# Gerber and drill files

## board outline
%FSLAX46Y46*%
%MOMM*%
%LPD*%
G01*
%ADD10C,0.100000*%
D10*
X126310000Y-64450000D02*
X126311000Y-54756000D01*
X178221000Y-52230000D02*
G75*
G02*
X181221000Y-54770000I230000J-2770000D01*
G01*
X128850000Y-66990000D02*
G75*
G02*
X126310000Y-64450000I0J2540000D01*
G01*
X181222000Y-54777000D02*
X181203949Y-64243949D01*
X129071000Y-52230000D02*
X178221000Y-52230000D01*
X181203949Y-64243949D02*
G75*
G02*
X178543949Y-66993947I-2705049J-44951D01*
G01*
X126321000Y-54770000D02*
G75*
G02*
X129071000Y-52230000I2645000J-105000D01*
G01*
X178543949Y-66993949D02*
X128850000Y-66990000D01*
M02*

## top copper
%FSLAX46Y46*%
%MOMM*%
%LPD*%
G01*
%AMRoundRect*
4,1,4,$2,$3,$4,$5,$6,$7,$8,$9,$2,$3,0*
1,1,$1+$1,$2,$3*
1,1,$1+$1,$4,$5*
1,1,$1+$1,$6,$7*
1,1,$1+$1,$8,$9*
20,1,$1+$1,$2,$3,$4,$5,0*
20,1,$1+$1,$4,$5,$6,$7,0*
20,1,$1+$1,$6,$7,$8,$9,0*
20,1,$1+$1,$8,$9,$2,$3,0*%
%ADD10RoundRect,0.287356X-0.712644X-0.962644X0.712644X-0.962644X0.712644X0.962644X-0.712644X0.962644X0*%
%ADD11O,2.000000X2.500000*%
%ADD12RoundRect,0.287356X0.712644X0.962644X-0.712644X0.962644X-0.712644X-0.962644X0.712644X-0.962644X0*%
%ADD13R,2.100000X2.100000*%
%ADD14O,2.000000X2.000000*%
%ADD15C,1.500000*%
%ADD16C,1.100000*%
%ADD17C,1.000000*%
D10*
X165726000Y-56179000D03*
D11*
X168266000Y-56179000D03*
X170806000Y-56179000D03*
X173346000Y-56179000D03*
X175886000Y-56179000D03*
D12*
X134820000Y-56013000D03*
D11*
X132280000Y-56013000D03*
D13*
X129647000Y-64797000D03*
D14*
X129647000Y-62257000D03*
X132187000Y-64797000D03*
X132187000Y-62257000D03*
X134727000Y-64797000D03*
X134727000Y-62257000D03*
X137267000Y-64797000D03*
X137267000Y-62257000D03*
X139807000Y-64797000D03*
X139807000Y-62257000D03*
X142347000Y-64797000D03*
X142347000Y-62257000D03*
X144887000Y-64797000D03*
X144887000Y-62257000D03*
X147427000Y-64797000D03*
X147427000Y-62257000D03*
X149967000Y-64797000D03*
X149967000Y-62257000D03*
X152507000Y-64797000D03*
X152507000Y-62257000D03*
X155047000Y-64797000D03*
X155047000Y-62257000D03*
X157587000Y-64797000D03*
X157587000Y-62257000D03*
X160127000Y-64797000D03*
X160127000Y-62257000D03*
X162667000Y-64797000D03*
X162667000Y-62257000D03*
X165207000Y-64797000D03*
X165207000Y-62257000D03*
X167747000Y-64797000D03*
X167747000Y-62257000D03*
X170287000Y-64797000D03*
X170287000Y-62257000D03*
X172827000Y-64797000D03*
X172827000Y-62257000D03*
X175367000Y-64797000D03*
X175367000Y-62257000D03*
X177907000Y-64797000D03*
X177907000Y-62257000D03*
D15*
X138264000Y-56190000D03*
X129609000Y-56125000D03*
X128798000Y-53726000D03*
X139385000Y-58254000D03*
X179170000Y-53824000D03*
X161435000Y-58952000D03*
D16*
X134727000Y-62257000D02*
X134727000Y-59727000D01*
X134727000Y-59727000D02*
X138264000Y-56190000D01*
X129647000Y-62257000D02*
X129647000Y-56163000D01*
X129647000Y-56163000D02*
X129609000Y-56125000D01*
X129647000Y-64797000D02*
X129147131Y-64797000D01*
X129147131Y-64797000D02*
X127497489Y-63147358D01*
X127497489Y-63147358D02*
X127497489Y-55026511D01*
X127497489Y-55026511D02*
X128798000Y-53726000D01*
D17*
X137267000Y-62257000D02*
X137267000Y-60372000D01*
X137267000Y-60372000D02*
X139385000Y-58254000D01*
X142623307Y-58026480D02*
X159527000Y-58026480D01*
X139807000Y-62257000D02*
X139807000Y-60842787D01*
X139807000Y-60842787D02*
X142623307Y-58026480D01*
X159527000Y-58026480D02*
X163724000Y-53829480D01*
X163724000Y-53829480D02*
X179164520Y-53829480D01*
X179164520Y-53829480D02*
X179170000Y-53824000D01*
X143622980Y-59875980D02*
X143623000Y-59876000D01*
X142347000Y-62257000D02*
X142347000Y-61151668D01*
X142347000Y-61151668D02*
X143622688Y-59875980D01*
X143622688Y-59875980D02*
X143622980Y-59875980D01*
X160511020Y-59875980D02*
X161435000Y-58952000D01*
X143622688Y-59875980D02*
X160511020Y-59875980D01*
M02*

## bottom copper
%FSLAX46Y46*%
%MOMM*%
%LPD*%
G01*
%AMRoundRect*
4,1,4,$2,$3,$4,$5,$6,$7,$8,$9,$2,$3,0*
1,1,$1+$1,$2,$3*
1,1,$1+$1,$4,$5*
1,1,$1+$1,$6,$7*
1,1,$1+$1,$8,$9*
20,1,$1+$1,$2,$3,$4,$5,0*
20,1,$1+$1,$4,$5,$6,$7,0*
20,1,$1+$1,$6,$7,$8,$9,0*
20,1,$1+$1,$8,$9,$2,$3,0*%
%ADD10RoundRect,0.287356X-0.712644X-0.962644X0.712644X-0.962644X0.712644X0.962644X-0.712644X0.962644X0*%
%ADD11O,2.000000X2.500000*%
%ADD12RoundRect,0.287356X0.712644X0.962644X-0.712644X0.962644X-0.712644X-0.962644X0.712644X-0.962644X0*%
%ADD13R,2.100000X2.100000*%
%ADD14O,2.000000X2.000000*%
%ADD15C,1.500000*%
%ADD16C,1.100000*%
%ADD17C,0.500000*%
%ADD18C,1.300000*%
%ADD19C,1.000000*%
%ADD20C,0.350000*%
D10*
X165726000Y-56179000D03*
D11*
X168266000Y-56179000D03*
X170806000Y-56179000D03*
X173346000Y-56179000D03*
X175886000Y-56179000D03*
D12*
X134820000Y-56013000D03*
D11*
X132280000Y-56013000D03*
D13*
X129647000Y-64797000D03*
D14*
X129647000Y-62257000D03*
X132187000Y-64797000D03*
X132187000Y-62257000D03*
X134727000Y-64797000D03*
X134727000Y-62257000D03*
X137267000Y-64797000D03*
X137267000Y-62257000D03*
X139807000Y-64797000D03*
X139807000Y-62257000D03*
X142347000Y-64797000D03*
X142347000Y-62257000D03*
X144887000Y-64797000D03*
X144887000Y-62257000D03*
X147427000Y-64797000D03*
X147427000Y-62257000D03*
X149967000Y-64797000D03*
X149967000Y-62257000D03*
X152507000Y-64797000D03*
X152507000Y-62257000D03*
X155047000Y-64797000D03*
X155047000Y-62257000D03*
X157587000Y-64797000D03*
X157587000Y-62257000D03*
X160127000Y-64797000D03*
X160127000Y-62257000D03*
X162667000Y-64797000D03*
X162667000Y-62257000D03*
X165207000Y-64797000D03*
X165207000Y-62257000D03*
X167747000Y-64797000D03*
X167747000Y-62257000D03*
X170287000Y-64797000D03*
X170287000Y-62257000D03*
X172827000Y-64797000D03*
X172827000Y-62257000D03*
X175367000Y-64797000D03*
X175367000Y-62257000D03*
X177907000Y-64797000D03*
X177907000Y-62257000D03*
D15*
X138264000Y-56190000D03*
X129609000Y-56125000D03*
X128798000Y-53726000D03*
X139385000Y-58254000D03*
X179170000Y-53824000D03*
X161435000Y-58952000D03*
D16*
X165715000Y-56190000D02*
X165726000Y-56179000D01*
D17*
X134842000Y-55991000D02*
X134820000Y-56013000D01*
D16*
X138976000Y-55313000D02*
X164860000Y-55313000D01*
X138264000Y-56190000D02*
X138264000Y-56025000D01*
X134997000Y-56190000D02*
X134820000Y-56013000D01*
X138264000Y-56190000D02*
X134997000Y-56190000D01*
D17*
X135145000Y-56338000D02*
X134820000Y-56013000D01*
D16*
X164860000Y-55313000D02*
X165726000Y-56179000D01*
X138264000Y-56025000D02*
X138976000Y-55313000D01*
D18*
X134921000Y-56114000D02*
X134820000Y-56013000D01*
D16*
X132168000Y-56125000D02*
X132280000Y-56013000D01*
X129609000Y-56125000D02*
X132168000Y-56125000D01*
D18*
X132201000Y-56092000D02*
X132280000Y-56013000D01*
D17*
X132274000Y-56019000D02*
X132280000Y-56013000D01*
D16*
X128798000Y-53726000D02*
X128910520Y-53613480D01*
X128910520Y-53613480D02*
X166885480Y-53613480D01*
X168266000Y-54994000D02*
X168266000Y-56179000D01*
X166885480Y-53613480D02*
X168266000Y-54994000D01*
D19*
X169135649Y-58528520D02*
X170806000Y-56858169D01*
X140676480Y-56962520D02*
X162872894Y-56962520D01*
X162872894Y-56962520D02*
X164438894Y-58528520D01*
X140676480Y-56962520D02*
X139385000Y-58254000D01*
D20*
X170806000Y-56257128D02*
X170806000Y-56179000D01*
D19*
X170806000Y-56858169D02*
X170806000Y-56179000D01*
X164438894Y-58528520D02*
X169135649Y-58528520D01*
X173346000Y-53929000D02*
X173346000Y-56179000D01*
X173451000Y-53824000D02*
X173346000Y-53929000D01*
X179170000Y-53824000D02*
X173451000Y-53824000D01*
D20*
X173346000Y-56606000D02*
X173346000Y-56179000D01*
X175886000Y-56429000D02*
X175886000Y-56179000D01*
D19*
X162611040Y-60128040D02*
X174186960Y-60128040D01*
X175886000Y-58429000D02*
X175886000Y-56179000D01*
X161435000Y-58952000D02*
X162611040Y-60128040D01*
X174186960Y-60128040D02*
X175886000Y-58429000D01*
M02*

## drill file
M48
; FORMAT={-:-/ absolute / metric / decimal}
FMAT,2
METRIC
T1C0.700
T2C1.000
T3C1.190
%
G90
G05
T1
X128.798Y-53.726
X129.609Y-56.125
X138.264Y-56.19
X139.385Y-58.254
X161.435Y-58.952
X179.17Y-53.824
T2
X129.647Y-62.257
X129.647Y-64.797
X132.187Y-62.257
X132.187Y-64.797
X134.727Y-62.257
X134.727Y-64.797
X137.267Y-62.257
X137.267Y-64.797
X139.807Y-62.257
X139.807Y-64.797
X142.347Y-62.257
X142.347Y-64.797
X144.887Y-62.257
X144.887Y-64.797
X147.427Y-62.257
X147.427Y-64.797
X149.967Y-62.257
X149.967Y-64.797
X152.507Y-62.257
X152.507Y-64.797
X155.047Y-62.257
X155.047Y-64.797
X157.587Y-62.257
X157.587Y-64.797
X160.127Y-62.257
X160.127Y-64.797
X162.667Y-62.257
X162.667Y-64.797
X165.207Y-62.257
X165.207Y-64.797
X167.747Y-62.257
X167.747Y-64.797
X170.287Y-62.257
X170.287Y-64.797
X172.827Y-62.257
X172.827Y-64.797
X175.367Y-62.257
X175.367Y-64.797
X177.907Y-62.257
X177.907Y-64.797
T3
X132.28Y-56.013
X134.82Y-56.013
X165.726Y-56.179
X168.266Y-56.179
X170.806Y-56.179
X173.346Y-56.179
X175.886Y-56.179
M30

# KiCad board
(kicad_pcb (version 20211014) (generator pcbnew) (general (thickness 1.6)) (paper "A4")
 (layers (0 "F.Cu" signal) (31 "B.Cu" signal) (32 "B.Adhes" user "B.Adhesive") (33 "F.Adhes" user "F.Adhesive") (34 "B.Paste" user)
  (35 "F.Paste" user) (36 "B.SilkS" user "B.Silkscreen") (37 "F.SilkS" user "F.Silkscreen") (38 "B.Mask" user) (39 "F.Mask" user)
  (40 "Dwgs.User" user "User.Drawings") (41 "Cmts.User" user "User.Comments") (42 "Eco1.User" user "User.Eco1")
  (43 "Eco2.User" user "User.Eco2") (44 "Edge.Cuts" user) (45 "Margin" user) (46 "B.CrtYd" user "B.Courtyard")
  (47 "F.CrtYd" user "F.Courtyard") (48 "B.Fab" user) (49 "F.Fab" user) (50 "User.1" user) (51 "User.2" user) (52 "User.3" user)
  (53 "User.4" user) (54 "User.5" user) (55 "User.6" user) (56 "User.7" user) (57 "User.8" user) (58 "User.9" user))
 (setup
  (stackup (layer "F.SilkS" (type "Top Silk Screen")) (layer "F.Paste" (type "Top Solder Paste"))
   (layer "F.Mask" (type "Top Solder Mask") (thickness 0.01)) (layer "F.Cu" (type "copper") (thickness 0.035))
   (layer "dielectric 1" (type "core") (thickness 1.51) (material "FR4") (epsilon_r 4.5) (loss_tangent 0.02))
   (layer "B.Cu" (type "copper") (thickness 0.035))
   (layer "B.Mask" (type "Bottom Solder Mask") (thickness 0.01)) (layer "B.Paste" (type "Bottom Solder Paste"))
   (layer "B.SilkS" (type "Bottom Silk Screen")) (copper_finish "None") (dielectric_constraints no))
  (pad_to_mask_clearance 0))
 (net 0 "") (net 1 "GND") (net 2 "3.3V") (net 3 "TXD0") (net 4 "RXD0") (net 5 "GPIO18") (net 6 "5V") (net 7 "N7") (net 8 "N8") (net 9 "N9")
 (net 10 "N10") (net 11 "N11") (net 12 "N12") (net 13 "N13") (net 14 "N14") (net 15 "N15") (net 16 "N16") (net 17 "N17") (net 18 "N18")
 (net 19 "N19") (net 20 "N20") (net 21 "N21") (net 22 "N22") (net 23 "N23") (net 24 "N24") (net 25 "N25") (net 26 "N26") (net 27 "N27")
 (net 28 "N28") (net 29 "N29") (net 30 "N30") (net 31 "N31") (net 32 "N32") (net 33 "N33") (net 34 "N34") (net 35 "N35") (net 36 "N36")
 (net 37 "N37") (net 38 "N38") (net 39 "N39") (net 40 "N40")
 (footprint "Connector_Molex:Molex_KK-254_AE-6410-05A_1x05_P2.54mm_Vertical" (layer "F.Cu") (at 165.726 56.179)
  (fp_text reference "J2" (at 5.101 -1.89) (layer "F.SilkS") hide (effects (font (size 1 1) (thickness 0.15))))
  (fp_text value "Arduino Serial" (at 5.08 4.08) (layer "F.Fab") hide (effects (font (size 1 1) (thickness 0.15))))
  (pad "1" thru_hole roundrect (at 0 0) (size 2 2.5) (drill 1.19) (layers *.Cu *.Mask) (roundrect_rratio 0.143678) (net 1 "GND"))
  (pad "2" thru_hole oval (at 2.54 0) (size 2 2.5) (drill 1.19) (layers *.Cu *.Mask) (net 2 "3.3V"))
  (pad "3" thru_hole oval (at 5.08 0) (size 2 2.5) (drill 1.19) (layers *.Cu *.Mask) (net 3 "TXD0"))
  (pad "4" thru_hole oval (at 7.62 0) (size 2 2.5) (drill 1.19) (layers *.Cu *.Mask) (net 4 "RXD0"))
  (pad "5" thru_hole oval (at 10.16 0) (size 2 2.5) (drill 1.19) (layers *.Cu *.Mask) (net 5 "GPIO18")))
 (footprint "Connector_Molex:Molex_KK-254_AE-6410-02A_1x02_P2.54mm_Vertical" (layer "F.Cu") (at 134.82 56.013 180)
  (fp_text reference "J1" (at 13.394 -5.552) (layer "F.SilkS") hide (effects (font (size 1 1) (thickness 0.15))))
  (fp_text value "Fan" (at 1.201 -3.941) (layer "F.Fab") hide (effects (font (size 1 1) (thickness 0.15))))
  (pad "1" thru_hole roundrect (at 0 0 180) (size 2 2.5) (drill 1.19) (layers *.Cu *.Mask) (roundrect_rratio 0.143678) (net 1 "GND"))
  (pad "2" thru_hole oval (at 2.54 0 180) (size 2 2.5) (drill 1.19) (layers *.Cu *.Mask) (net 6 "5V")))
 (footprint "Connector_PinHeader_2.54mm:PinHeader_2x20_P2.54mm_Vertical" (layer "F.Cu") (at 129.647 64.797 90)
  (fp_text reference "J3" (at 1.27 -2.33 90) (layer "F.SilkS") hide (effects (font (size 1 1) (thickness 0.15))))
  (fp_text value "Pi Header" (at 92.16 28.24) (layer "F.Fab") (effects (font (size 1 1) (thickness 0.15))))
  (pad "1" thru_hole rect (at 0 0 90) (size 2.1 2.1) (drill 1) (layers *.Cu *.Mask) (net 2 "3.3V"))
  (pad "2" thru_hole oval (at 2.54 0 90) (size 2 2) (drill 1) (layers *.Cu *.Mask) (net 6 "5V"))
  (pad "3" thru_hole oval (at 0 2.54 90) (size 2 2) (drill 1) (layers *.Cu *.Mask) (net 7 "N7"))
  (pad "4" thru_hole oval (at 2.54 2.54 90) (size 2 2) (drill 1) (layers *.Cu *.Mask) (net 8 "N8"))
  (pad "5" thru_hole oval (at 0 5.08 90) (size 2 2) (drill 1) (layers *.Cu *.Mask) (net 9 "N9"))
  (pad "6" thru_hole oval (at 2.54 5.08 90) (size 2 2) (drill 1) (layers *.Cu *.Mask) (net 1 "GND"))
  (pad "7" thru_hole oval (at 0 7.62 90) (size 2 2) (drill 1) (layers *.Cu *.Mask) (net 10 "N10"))
  (pad "8" thru_hole oval (at 2.54 7.62 90) (size 2 2) (drill 1) (layers *.Cu *.Mask) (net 3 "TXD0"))
  (pad "9" thru_hole oval (at 0 10.16 90) (size 2 2) (drill 1) (layers *.Cu *.Mask) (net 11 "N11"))
  (pad "10" thru_hole oval (at 2.54 10.16 90) (size 2 2) (drill 1) (layers *.Cu *.Mask) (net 4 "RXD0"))
  (pad "11" thru_hole oval (at 0 12.7 90) (size 2 2) (drill 1) (layers *.Cu *.Mask) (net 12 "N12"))
  (pad "12" thru_hole oval (at 2.54 12.7 90) (size 2 2) (drill 1) (layers *.Cu *.Mask) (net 5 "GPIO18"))
  (pad "13" thru_hole oval (at 0 15.24 90) (size 2 2) (drill 1) (layers *.Cu *.Mask) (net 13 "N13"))
  (pad "14" thru_hole oval (at 2.54 15.24 90) (size 2 2) (drill 1) (layers *.Cu *.Mask) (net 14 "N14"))
  (pad "15" thru_hole oval (at 0 17.78 90) (size 2 2) (drill 1) (layers *.Cu *.Mask) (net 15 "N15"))
  (pad "16" thru_hole oval (at 2.54 17.78 90) (size 2 2) (drill 1) (layers *.Cu *.Mask) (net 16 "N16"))
  (pad "17" thru_hole oval (at 0 20.32 90) (size 2 2) (drill 1) (layers *.Cu *.Mask) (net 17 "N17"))
  (pad "18" thru_hole oval (at 2.54 20.32 90) (size 2 2) (drill 1) (layers *.Cu *.Mask) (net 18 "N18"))
  (pad "19" thru_hole oval (at 0 22.86 90) (size 2 2) (drill 1) (layers *.Cu *.Mask) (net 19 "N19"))
  (pad "20" thru_hole oval (at 2.54 22.86 90) (size 2 2) (drill 1) (layers *.Cu *.Mask) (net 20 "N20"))
  (pad "21" thru_hole oval (at 0 25.4 90) (size 2 2) (drill 1) (layers *.Cu *.Mask) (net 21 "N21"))
  (pad "22" thru_hole oval (at 2.54 25.4 90) (size 2 2) (drill 1) (layers *.Cu *.Mask) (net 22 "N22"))
  (pad "23" thru_hole oval (at 0 27.94 90) (size 2 2) (drill 1) (layers *.Cu *.Mask) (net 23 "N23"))
  (pad "24" thru_hole oval (at 2.54 27.94 90) (size 2 2) (drill 1) (layers *.Cu *.Mask) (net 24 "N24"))
  (pad "25" thru_hole oval (at 0 30.48 90) (size 2 2) (drill 1) (layers *.Cu *.Mask) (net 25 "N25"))
  (pad "26" thru_hole oval (at 2.54 30.48 90) (size 2 2) (drill 1) (layers *.Cu *.Mask) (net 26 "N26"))
  (pad "27" thru_hole oval (at 0 33.02 90) (size 2 2) (drill 1) (layers *.Cu *.Mask) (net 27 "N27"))
  (pad "28" thru_hole oval (at 2.54 33.02 90) (size 2 2) (drill 1) (layers *.Cu *.Mask) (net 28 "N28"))
  (pad "29" thru_hole oval (at 0 35.56 90) (size 2 2) (drill 1) (layers *.Cu *.Mask) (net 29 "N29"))
  (pad "30" thru_hole oval (at 2.54 35.56 90) (size 2 2) (drill 1) (layers *.Cu *.Mask) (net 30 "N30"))
  (pad "31" thru_hole oval (at 0 38.1 90) (size 2 2) (drill 1) (layers *.Cu *.Mask) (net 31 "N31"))
  (pad "32" thru_hole oval (at 2.54 38.1 90) (size 2 2) (drill 1) (layers *.Cu *.Mask) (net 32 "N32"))
  (pad "33" thru_hole oval (at 0 40.64 90) (size 2 2) (drill 1) (layers *.Cu *.Mask) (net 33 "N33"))
  (pad "34" thru_hole oval (at 2.54 40.64 90) (size 2 2) (drill 1) (layers *.Cu *.Mask) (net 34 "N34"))
  (pad "35" thru_hole oval (at 0 43.18 90) (size 2 2) (drill 1) (layers *.Cu *.Mask) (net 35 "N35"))
  (pad "36" thru_hole oval (at 2.54 43.18 90) (size 2 2) (drill 1) (layers *.Cu *.Mask) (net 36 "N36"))
  (pad "37" thru_hole oval (at 0 45.72 90) (size 2 2) (drill 1) (layers *.Cu *.Mask) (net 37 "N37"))
  (pad "38" thru_hole oval (at 2.54 45.72 90) (size 2 2) (drill 1) (layers *.Cu *.Mask) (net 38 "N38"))
  (pad "39" thru_hole oval (at 0 48.26 90) (size 2 2) (drill 1) (layers *.Cu *.Mask) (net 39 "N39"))
  (pad "40" thru_hole oval (at 2.54 48.26 90) (size 2 2) (drill 1) (layers *.Cu *.Mask) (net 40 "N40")))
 (gr_line (start 126.31 64.45) (end 126.311 54.756) (layer "Edge.Cuts") (width 0.1))
 (gr_arc (start 178.221 52.23) (mid 180.247051 52.87868) (end 181.221 54.77) (layer "Edge.Cuts") (width 0.1))
 (gr_arc (start 128.85 66.99) (mid 127.053949 66.246051) (end 126.31 64.45) (layer "Edge.Cuts") (width 0.1))
 (gr_line (start 181.222 54.777) (end 181.203949 64.243949) (layer "Edge.Cuts") (width 0.1))
 (gr_line (start 129.071 52.23) (end 178.221 52.23) (layer "Edge.Cuts") (width 0.1))
 (gr_arc (start 181.203949 64.243949) (mid 180.443493 66.169853) (end 178.543949 66.993949) (layer "Edge.Cuts") (width 0.1))
 (gr_arc (start 126.321 54.77) (mid 127.169949 52.930456) (end 129.071 52.23) (layer "Edge.Cuts") (width 0.1))
 (gr_line (start 178.543949 66.993949) (end 128.85 66.99) (layer "Edge.Cuts") (width 0.1))
 (segment (start 134.727 62.257) (end 134.727 59.727) (width 1.1) (layer "F.Cu") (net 1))
 (segment (start 134.727 59.727) (end 138.264 56.19) (width 1.1) (layer "F.Cu") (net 1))
 (via (at 138.264 56.19) (size 1.5) (drill 0.7) (layers "F.Cu" "B.Cu") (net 1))
 (segment (start 165.715 56.19) (end 165.726 56.179) (width 1.1) (layer "B.Cu") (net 1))
 (segment (start 134.842 55.991) (end 134.82 56.013) (width 0.5) (layer "B.Cu") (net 1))
 (segment (start 138.976 55.313) (end 164.86 55.313) (width 1.1) (layer "B.Cu") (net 1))
 (segment (start 138.264 56.19) (end 138.264 56.025) (width 1.1) (layer "B.Cu") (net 1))
 (segment (start 134.997 56.19) (end 134.82 56.013) (width 1.1) (layer "B.Cu") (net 1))
 (segment (start 138.264 56.19) (end 134.997 56.19) (width 1.1) (layer "B.Cu") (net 1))
 (segment (start 135.145 56.338) (end 134.82 56.013) (width 0.5) (layer "B.Cu") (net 1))
 (segment (start 164.86 55.313) (end 165.726 56.179) (width 1.1) (layer "B.Cu") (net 1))
 (segment (start 138.264 56.025) (end 138.976 55.313) (width 1.1) (layer "B.Cu") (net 1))
 (segment (start 134.921 56.114) (end 134.82 56.013) (width 1.3) (layer "B.Cu") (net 1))
 (segment (start 129.647 62.257) (end 129.647 56.163) (width 1.1) (layer "F.Cu") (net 6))
 (segment (start 129.647 56.163) (end 129.609 56.125) (width 1.1) (layer "F.Cu") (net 6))
 (via (at 129.609 56.125) (size 1.5) (drill 0.7) (layers "F.Cu" "B.Cu") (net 6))
 (segment (start 132.168 56.125) (end 132.28 56.013) (width 1.1) (layer "B.Cu") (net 6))
 (segment (start 129.609 56.125) (end 132.168 56.125) (width 1.1) (layer "B.Cu") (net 6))
 (segment (start 132.201 56.092) (end 132.28 56.013) (width 1.3) (layer "B.Cu") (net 6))
 (segment (start 132.274 56.019) (end 132.28 56.013) (width 0.5) (layer "B.Cu") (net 6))
 (segment (start 129.647 64.797) (end 129.147131 64.797) (width 1.1) (layer "F.Cu") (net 2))
 (segment (start 129.147131 64.797) (end 127.497489 63.147358) (width 1.1) (layer "F.Cu") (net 2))
 (segment (start 127.497489 63.147358) (end 127.497489 55.026511) (width 1.1) (layer "F.Cu") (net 2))
 (segment (start 127.497489 55.026511) (end 128.798 53.726) (width 1.1) (layer "F.Cu") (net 2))
 (via (at 128.798 53.726) (size 1.5) (drill 0.7) (layers "F.Cu" "B.Cu") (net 2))
 (segment (start 128.798 53.726) (end 128.91052 53.61348) (width 1.1) (layer "B.Cu") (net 2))
 (segment (start 128.91052 53.61348) (end 166.88548 53.61348) (width 1.1) (layer "B.Cu") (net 2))
 (segment (start 168.266 54.994) (end 168.266 56.179) (width 1.1) (layer "B.Cu") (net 2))
 (segment (start 166.88548 53.61348) (end 168.266 54.994) (width 1.1) (layer "B.Cu") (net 2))
 (segment (start 137.267 62.257) (end 137.267 60.372) (width 1) (layer "F.Cu") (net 3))
 (segment (start 137.267 60.372) (end 139.385 58.254) (width 1) (layer "F.Cu") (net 3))
 (via (at 139.385 58.254) (size 1.5) (drill 0.7) (layers "F.Cu" "B.Cu") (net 3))
 (segment (start 169.135649 58.52852) (end 170.806 56.858169) (width 1) (layer "B.Cu") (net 3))
 (segment (start 140.67648 56.96252) (end 162.872894 56.96252) (width 1) (layer "B.Cu") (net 3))
 (segment (start 162.872894 56.96252) (end 164.438894 58.52852) (width 1) (layer "B.Cu") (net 3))
 (segment (start 140.67648 56.96252) (end 139.385 58.254) (width 1) (layer "B.Cu") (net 3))
 (segment (start 170.806 56.257128) (end 170.806 56.179) (width 0.35) (layer "B.Cu") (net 3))
 (segment (start 170.806 56.858169) (end 170.806 56.179) (width 1) (layer "B.Cu") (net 3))
 (segment (start 164.438894 58.52852) (end 169.135649 58.52852) (width 1) (layer "B.Cu") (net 3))
 (segment (start 142.623307 58.02648) (end 159.527 58.02648) (width 1) (layer "F.Cu") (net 4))
 (segment (start 139.807 62.257) (end 139.807 60.842787) (width 1) (layer "F.Cu") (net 4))
 (segment (start 139.807 60.842787) (end 142.623307 58.02648) (width 1) (layer "F.Cu") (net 4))
 (segment (start 159.527 58.02648) (end 163.724 53.82948) (width 1) (layer "F.Cu") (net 4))
 (segment (start 163.724 53.82948) (end 179.16452 53.82948) (width 1) (layer "F.Cu") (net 4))
 (segment (start 179.16452 53.82948) (end 179.17 53.824) (width 1) (layer "F.Cu") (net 4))
 (via (at 179.17 53.824) (size 1.5) (drill 0.7) (layers "F.Cu" "B.Cu") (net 4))
 (segment (start 173.346 53.929) (end 173.346 56.179) (width 1) (layer "B.Cu") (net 4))
 (segment (start 173.451 53.824) (end 173.346 53.929) (width 1) (layer "B.Cu") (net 4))
 (segment (start 179.17 53.824) (end 173.451 53.824) (width 1) (layer "B.Cu") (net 4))
 (segment (start 173.346 56.606) (end 173.346 56.179) (width 0.35) (layer "B.Cu") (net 4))
 (segment (start 143.62298 59.87598) (end 143.623 59.876) (width 1) (layer "F.Cu") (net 5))
 (segment (start 142.347 62.257) (end 142.347 61.151668) (width 1) (layer "F.Cu") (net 5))
 (segment (start 142.347 61.151668) (end 143.622688 59.87598) (width 1) (layer "F.Cu") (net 5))
 (segment (start 143.622688 59.87598) (end 143.62298 59.87598) (width 1) (layer "F.Cu") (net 5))
 (segment (start 160.51102 59.87598) (end 161.435 58.952) (width 1) (layer "F.Cu") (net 5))
 (segment (start 143.622688 59.87598) (end 160.51102 59.87598) (width 1) (layer "F.Cu") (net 5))
 (via (at 161.435 58.952) (size 1.5) (drill 0.7) (layers "F.Cu" "B.Cu") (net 5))
 (segment (start 175.886 56.429) (end 175.886 56.179) (width 0.35) (layer "B.Cu") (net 5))
 (segment (start 162.61104 60.12804) (end 174.18696 60.12804) (width 1) (layer "B.Cu") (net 5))
 (segment (start 175.886 58.429) (end 175.886 56.179) (width 1) (layer "B.Cu") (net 5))
 (segment (start 161.435 58.952) (end 162.61104 60.12804) (width 1) (layer "B.Cu") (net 5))
 (segment (start 174.18696 60.12804) (end 175.886 58.429) (width 1) (layer "B.Cu") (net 5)))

